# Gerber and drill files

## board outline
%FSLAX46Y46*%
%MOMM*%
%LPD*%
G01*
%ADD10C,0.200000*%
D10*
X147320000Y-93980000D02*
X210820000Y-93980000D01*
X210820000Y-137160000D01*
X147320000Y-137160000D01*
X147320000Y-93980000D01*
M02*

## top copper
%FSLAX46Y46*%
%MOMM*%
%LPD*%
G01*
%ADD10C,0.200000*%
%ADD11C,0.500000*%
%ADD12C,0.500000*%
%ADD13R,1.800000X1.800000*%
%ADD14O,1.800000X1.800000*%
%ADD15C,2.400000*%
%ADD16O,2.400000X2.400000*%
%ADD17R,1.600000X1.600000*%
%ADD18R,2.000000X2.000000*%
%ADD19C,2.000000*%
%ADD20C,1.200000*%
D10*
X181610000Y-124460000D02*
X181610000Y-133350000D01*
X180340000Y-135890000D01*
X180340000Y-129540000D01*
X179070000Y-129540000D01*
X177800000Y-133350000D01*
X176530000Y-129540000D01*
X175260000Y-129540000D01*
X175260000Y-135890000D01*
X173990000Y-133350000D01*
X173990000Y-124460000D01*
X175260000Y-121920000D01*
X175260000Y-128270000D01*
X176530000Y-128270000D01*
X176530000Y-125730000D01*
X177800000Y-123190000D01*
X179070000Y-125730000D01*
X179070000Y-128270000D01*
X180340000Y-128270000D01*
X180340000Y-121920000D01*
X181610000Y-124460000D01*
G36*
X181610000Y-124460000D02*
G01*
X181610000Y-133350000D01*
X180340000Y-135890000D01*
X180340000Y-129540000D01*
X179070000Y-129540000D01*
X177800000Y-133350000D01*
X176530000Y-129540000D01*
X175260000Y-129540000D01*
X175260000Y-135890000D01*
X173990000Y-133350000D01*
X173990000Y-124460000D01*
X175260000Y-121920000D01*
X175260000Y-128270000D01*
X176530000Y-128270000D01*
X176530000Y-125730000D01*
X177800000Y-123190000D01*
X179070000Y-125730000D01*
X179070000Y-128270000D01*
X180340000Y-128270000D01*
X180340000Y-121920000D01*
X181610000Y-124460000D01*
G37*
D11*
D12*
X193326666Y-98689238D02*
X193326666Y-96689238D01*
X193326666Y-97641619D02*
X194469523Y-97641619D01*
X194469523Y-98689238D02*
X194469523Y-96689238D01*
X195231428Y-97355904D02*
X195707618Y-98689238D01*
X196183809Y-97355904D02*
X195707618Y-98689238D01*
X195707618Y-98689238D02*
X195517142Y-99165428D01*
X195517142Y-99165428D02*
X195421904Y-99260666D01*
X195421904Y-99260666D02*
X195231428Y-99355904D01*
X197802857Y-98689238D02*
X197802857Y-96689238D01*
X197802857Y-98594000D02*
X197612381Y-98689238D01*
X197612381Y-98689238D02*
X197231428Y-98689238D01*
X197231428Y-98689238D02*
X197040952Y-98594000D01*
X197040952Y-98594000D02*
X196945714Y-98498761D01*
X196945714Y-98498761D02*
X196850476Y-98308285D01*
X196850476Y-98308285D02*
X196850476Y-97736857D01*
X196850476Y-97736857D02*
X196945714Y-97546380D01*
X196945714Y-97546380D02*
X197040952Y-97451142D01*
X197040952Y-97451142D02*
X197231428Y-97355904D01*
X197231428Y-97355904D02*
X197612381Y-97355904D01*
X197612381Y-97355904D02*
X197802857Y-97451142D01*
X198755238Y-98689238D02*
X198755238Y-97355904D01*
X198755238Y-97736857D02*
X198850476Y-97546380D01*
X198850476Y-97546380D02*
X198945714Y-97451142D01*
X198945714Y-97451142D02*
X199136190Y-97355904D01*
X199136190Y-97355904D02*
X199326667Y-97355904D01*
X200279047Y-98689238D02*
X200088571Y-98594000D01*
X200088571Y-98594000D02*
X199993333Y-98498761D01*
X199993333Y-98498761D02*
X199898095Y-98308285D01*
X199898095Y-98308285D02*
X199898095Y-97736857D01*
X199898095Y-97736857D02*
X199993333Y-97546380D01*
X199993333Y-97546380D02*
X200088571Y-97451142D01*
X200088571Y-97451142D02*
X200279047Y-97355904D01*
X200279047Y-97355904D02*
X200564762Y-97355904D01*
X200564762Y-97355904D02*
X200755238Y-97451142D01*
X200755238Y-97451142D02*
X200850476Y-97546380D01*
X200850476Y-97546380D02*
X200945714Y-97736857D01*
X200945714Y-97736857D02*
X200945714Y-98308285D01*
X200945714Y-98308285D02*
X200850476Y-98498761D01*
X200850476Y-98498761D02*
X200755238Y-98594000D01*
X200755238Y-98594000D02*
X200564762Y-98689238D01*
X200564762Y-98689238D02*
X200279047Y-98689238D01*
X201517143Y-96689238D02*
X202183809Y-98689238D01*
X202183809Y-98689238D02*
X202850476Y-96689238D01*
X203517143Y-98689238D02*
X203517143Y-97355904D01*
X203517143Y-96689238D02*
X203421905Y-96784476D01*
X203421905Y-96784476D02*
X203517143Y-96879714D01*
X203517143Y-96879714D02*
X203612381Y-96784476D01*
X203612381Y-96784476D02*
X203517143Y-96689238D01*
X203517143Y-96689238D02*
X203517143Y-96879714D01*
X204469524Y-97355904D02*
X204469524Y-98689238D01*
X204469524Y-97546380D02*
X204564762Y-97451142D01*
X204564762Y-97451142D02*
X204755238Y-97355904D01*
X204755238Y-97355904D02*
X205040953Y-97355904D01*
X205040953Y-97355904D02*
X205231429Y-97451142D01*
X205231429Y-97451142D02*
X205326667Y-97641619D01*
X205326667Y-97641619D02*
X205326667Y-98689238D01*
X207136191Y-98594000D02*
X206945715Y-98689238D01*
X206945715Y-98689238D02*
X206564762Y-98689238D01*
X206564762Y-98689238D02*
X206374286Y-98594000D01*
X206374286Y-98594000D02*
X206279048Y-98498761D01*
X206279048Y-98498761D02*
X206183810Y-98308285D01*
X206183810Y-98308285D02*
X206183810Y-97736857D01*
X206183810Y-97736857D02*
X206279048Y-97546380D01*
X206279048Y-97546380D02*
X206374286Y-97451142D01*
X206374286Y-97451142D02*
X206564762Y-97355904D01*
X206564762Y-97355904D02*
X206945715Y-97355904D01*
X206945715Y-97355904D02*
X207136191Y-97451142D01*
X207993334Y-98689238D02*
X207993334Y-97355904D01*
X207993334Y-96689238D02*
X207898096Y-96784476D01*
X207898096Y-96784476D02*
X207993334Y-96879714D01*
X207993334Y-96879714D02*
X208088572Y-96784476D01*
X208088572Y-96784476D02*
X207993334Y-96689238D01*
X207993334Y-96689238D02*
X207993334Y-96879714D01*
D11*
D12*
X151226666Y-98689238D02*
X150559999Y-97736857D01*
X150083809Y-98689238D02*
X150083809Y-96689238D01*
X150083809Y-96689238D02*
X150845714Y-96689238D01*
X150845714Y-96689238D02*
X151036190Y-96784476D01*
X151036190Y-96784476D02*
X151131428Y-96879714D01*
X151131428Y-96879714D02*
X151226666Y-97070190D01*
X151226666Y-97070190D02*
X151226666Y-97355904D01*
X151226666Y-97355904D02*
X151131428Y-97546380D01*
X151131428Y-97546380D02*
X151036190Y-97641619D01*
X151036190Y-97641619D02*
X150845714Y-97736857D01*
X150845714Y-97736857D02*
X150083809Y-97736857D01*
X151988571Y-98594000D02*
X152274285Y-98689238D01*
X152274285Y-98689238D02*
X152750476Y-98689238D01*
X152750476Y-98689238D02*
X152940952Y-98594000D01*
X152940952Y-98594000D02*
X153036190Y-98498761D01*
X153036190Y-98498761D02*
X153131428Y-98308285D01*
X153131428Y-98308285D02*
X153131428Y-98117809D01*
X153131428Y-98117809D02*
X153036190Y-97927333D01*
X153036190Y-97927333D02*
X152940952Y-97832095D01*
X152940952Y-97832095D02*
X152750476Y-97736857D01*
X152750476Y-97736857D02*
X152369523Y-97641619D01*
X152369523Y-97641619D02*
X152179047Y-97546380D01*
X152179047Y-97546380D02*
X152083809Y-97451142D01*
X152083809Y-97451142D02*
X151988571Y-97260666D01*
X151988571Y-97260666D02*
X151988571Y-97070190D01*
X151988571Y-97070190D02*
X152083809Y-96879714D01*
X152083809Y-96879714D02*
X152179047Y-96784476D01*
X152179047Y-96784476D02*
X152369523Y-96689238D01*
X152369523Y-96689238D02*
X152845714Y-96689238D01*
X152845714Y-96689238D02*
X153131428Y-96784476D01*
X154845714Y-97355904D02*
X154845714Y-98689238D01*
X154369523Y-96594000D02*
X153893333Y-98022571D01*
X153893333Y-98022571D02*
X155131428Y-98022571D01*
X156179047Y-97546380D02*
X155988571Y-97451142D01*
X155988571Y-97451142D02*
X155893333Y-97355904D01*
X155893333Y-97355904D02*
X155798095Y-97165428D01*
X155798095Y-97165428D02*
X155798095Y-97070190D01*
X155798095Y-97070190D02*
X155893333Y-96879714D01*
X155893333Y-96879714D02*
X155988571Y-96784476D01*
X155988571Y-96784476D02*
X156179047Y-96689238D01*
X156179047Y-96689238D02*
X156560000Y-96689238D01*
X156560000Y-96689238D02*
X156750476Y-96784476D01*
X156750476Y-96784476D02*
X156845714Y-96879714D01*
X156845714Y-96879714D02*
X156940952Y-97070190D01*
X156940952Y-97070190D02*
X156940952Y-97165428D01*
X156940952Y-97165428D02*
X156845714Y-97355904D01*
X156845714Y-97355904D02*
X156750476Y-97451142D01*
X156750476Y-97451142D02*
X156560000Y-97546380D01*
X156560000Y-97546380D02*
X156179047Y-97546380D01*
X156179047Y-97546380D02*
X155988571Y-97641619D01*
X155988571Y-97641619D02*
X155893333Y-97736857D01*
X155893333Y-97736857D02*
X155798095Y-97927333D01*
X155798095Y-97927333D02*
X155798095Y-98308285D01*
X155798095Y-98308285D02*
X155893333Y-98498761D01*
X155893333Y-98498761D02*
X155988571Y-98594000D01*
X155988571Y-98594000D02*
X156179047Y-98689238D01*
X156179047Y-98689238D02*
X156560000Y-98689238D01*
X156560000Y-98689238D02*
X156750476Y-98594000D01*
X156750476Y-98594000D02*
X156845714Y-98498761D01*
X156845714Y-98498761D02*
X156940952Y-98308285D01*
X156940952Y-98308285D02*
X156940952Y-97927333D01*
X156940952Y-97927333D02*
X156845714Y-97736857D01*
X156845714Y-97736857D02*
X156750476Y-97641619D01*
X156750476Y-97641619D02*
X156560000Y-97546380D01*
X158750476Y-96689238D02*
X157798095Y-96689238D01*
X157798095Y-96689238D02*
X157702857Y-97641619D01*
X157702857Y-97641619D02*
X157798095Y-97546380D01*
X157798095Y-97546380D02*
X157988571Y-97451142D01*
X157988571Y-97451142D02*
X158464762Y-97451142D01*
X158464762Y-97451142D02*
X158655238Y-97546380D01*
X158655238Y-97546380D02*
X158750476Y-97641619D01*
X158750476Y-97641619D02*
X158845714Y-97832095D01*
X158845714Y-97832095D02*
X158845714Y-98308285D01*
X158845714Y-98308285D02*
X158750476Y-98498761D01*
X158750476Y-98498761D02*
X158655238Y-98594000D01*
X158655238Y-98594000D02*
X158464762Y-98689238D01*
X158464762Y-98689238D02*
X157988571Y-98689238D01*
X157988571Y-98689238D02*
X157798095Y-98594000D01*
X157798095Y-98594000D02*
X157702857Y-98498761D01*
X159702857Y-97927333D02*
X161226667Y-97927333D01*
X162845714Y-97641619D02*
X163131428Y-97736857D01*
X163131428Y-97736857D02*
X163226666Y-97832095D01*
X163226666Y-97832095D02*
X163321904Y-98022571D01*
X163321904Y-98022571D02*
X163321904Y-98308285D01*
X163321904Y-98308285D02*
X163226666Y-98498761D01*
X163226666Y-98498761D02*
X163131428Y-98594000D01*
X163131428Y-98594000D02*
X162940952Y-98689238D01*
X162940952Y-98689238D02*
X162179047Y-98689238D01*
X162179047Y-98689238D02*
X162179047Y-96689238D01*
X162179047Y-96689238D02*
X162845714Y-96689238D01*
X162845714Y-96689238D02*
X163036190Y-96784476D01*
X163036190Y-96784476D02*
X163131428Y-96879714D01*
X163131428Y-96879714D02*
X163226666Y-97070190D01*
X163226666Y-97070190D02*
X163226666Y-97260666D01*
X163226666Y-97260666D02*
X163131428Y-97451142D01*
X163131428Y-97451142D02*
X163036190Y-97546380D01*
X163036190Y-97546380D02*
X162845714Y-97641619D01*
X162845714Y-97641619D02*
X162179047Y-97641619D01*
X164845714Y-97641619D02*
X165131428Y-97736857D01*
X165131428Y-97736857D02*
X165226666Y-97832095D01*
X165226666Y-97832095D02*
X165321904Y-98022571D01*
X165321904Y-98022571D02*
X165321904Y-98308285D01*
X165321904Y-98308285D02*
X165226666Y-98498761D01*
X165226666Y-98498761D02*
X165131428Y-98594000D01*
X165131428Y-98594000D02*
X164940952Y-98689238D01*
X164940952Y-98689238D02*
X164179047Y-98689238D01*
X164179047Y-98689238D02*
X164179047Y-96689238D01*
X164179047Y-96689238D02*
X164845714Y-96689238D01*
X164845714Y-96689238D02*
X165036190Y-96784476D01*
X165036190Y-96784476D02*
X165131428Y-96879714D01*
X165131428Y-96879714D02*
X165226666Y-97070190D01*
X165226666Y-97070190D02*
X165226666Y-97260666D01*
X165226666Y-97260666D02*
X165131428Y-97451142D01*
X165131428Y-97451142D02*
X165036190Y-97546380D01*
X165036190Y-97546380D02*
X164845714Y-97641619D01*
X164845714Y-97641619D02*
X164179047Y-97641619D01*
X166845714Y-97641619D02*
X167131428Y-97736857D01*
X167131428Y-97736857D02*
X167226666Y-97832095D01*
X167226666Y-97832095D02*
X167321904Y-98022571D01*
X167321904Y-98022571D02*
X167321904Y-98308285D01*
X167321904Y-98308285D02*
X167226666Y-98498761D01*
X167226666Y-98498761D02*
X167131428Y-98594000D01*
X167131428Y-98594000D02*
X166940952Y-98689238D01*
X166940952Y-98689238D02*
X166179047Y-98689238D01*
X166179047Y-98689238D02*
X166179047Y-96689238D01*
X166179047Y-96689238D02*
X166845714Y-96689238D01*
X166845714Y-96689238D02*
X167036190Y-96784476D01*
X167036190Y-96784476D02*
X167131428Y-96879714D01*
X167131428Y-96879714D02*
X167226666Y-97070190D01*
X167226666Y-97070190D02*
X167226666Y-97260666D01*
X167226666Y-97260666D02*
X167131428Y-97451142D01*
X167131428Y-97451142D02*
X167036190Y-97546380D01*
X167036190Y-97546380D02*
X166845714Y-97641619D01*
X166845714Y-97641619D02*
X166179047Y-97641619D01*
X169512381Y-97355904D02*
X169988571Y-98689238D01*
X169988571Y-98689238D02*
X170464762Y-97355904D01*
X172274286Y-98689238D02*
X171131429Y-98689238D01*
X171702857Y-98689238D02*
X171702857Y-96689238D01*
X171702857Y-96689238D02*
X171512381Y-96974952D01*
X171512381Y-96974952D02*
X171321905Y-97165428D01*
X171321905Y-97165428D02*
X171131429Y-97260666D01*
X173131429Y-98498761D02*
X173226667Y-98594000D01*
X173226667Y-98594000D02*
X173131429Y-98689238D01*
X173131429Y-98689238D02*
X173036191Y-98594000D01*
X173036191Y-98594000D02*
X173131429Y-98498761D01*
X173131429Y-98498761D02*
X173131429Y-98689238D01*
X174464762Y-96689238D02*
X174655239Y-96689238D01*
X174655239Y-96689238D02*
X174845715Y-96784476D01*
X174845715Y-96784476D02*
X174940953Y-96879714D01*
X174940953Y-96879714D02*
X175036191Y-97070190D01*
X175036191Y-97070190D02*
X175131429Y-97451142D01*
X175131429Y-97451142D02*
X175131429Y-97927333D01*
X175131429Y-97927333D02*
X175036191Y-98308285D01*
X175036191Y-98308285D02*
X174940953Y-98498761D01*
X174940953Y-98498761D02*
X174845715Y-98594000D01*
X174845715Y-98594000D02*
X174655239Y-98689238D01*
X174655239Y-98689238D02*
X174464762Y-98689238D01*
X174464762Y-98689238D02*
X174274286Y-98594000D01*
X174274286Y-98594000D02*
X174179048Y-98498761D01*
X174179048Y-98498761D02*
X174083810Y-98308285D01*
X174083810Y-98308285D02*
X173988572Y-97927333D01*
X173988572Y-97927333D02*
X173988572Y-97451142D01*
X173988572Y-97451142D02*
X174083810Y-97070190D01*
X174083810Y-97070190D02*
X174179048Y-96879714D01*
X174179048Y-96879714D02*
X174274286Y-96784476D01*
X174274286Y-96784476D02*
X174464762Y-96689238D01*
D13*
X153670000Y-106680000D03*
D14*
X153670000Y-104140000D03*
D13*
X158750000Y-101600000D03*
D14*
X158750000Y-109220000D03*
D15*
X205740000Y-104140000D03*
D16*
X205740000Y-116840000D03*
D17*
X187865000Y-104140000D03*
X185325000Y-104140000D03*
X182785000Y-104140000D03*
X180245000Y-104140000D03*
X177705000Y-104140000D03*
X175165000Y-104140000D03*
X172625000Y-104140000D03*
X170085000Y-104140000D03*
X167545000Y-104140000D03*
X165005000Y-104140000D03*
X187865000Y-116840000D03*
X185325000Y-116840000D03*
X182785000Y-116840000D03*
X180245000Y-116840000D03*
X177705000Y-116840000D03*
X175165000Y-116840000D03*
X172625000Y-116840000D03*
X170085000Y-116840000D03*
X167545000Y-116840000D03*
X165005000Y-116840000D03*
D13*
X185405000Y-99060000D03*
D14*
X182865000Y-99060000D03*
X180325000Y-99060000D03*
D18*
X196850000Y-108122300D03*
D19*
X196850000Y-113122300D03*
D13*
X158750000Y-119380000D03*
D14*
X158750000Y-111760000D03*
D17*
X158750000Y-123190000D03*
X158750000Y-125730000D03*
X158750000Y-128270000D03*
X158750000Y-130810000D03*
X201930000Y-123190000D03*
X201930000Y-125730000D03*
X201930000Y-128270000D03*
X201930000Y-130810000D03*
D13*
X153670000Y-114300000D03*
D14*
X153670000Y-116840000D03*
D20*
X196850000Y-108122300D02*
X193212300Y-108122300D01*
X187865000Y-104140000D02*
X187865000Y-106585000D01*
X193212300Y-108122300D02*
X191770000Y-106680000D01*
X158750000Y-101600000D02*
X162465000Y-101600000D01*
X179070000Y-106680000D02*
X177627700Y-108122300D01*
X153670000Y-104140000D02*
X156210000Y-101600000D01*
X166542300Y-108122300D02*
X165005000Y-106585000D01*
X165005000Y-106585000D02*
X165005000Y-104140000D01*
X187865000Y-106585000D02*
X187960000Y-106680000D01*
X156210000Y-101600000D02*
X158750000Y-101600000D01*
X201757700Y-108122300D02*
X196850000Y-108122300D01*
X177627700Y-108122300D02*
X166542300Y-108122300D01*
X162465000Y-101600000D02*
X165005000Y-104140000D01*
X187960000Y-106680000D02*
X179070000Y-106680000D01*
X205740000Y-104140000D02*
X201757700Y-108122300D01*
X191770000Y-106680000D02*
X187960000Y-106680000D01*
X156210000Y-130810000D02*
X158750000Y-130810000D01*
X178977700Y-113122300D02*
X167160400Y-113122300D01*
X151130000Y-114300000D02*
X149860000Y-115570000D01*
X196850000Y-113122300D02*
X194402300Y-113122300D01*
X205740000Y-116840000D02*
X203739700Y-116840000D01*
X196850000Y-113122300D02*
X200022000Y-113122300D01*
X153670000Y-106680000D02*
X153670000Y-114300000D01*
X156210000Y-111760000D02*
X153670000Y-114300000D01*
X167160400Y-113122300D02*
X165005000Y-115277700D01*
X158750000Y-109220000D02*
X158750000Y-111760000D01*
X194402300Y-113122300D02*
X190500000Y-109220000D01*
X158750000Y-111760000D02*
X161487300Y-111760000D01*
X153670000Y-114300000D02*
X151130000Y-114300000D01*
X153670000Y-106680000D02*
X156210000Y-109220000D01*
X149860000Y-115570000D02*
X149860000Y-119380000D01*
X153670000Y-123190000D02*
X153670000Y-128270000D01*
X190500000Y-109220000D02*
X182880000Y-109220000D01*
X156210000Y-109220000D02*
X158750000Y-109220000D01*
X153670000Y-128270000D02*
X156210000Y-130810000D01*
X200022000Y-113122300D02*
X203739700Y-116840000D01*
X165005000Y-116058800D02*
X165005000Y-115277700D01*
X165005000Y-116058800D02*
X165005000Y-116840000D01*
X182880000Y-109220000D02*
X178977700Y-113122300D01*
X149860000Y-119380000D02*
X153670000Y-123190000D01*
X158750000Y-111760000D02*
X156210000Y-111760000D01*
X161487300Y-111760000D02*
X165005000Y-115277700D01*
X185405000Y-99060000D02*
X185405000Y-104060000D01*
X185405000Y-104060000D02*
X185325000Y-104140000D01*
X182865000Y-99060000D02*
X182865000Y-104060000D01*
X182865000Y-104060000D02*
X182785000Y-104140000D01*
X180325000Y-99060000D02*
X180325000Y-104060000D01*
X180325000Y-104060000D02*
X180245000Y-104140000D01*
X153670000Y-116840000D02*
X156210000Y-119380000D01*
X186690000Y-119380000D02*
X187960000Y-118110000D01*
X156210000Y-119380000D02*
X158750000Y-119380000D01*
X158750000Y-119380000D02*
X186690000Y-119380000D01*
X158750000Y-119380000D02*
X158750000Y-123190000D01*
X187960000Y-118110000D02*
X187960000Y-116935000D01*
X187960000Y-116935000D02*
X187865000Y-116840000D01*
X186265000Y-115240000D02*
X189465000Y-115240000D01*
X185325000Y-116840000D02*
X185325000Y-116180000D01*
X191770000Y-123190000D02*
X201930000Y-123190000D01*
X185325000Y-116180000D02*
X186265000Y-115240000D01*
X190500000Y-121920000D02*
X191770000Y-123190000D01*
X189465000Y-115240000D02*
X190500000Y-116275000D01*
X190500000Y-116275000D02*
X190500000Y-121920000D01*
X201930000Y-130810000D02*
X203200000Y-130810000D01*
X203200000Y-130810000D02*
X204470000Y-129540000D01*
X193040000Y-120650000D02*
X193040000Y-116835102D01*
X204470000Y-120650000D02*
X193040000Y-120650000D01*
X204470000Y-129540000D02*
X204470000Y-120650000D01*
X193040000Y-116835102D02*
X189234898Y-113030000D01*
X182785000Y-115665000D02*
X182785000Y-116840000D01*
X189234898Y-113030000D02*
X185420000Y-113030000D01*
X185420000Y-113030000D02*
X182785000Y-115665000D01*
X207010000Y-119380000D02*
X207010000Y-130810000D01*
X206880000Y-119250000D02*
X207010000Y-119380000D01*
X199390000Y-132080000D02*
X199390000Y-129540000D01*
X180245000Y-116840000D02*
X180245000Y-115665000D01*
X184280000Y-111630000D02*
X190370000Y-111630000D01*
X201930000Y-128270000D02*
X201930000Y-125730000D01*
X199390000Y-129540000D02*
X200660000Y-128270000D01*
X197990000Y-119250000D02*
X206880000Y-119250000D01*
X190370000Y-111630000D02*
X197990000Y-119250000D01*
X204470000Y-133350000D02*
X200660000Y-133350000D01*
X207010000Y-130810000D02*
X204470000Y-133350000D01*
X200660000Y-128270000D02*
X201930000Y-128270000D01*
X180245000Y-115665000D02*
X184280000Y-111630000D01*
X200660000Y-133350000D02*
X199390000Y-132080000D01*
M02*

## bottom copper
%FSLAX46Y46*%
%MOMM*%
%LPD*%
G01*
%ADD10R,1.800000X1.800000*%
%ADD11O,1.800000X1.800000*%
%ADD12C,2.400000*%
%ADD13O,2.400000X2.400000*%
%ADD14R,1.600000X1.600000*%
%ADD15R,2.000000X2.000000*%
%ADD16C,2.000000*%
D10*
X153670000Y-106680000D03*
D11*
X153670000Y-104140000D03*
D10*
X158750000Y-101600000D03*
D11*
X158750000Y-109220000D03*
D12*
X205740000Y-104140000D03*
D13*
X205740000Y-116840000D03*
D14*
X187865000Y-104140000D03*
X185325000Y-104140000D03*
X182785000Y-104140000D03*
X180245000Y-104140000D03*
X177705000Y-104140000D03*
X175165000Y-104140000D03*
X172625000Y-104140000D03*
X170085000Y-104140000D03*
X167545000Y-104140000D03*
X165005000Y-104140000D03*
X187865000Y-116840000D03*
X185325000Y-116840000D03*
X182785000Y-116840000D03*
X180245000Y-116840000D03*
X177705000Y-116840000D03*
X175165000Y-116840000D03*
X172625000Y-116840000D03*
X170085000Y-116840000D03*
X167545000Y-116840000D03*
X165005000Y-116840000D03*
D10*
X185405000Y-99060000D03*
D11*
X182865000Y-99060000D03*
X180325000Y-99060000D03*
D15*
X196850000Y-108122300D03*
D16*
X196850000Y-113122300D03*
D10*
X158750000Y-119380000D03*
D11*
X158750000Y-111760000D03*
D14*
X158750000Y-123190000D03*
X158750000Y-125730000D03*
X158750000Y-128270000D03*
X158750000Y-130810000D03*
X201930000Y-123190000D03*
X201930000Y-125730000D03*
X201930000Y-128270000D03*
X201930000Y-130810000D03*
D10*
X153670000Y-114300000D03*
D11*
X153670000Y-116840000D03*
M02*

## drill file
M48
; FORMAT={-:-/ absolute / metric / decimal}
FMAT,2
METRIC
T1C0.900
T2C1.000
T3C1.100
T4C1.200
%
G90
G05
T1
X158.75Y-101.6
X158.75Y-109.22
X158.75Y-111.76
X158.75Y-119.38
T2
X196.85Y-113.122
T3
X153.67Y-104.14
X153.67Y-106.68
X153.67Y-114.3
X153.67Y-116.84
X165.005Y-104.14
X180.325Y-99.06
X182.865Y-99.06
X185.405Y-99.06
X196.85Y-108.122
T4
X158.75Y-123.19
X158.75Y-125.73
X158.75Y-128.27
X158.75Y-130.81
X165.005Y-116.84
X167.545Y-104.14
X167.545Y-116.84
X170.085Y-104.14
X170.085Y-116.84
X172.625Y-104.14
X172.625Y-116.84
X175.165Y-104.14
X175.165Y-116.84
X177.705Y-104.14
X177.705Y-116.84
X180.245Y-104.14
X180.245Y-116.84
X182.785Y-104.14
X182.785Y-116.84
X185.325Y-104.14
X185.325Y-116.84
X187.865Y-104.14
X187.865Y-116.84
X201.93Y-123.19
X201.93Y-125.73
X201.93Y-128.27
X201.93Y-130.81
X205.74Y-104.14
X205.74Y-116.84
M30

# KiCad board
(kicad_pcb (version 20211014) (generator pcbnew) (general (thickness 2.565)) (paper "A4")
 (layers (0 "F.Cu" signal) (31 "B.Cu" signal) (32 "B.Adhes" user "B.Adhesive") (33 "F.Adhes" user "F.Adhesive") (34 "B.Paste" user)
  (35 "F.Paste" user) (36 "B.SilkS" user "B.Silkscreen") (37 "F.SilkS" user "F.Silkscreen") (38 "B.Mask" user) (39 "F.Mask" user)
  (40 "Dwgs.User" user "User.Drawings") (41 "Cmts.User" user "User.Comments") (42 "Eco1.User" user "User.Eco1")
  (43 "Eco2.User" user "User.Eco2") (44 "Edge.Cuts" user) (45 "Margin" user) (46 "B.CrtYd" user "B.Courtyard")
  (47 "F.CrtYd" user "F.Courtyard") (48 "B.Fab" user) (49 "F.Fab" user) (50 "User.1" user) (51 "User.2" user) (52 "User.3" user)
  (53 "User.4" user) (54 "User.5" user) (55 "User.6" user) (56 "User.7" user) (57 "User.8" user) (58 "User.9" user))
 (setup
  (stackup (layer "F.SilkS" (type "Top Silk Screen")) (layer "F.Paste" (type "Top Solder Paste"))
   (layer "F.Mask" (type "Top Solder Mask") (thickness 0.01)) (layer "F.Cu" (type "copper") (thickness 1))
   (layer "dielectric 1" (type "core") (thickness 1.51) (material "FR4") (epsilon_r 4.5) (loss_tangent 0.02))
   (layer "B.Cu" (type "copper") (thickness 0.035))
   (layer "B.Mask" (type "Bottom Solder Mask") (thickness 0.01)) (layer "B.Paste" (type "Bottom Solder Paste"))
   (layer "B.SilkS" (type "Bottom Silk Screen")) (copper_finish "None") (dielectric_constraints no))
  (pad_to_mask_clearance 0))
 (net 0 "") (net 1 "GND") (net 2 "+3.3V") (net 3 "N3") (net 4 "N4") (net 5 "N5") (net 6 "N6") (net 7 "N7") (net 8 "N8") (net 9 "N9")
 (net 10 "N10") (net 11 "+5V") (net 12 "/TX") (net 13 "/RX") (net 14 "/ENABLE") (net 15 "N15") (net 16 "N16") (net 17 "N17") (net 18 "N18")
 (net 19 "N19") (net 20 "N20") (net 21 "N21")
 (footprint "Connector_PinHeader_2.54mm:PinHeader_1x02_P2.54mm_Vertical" (layer "F.Cu") (at 153.67 106.68 180)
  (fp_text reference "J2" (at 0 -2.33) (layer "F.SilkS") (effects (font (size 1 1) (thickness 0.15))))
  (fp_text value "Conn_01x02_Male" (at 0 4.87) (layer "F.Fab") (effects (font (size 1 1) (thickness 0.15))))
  (pad "1" thru_hole rect (at 0 0 180) (size 1.8 1.8) (drill 1.1) (layers *.Cu *.Mask) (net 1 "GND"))
  (pad "2" thru_hole oval (at 0 2.54 180) (size 1.8 1.8) (drill 1.1) (layers *.Cu *.Mask) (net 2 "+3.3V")))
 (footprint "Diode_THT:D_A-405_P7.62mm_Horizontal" (layer "F.Cu") (at 158.75 101.6 -90)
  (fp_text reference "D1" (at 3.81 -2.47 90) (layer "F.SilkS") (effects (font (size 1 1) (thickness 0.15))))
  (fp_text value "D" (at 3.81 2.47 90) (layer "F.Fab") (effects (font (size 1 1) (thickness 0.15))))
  (pad "1" thru_hole rect (at 0 0 270) (size 1.8 1.8) (drill 0.9) (layers *.Cu *.Mask) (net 2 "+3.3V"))
  (pad "2" thru_hole oval (at 7.62 0 270) (size 1.8 1.8) (drill 0.9) (layers *.Cu *.Mask) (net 1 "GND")))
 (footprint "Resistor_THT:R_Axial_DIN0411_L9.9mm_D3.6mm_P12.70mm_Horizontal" (layer "F.Cu") (at 205.74 104.14 -90)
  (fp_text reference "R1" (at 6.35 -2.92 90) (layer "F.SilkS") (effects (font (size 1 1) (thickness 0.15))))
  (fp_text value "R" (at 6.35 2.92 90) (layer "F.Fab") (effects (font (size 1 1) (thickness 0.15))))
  (pad "1" thru_hole circle (at 0 0 270) (size 2.4 2.4) (drill 1.2) (layers *.Cu *.Mask) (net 2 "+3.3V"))
  (pad "2" thru_hole oval (at 12.7 0 270) (size 2.4 2.4) (drill 1.2) (layers *.Cu *.Mask) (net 1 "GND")))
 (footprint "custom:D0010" (layer "F.Cu") (at 190.405 109.22 -90)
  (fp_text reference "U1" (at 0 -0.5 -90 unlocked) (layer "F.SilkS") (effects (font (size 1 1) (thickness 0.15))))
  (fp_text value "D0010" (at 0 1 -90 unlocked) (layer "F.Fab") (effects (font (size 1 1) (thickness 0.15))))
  (pad "1" thru_hole rect (at -5.08 2.54 270) (size 1.6 1.6) (drill 1.2) (layers *.Cu *.Mask) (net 2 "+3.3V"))
  (pad "2" thru_hole rect (at -5.08 5.08 270) (size 1.6 1.6) (drill 1.2) (layers *.Cu *.Mask) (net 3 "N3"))
  (pad "3" thru_hole rect (at -5.08 7.62 270) (size 1.6 1.6) (drill 1.2) (layers *.Cu *.Mask) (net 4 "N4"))
  (pad "4" thru_hole rect (at -5.08 10.16 270) (size 1.6 1.6) (drill 1.2) (layers *.Cu *.Mask) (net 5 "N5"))
  (pad "5" thru_hole rect (at -5.08 12.7 270) (size 1.6 1.6) (drill 1.2) (layers *.Cu *.Mask) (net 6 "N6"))
  (pad "6" thru_hole rect (at -5.08 15.24 270) (size 1.6 1.6) (drill 1.2) (layers *.Cu *.Mask) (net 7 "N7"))
  (pad "7" thru_hole rect (at -5.08 17.78 270) (size 1.6 1.6) (drill 1.2) (layers *.Cu *.Mask) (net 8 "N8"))
  (pad "8" thru_hole rect (at -5.08 20.32 270) (size 1.6 1.6) (drill 1.2) (layers *.Cu *.Mask) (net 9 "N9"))
  (pad "9" thru_hole rect (at -5.08 22.86 270) (size 1.6 1.6) (drill 1.2) (layers *.Cu *.Mask) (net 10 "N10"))
  (pad "10" thru_hole rect (at -5.08 25.4 270) (size 1.6 1.6) (drill 1.1) (layers *.Cu *.Mask) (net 2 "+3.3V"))
  (pad "11" thru_hole rect (at 7.62 2.54 270) (size 1.6 1.6) (drill 1.2) (layers *.Cu *.Mask) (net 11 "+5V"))
  (pad "12" thru_hole rect (at 7.62 5.08 270) (size 1.6 1.6) (drill 1.2) (layers *.Cu *.Mask) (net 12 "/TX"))
  (pad "13" thru_hole rect (at 7.62 7.62 270) (size 1.6 1.6) (drill 1.2) (layers *.Cu *.Mask) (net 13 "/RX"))
  (pad "14" thru_hole rect (at 7.62 10.16 270) (size 1.6 1.6) (drill 1.2) (layers *.Cu *.Mask) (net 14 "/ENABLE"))
  (pad "15" thru_hole rect (at 7.62 12.7 270) (size 1.6 1.6) (drill 1.2) (layers *.Cu *.Mask) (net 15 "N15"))
  (pad "16" thru_hole rect (at 7.62 15.24 270) (size 1.6 1.6) (drill 1.2) (layers *.Cu *.Mask) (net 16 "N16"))
  (pad "17" thru_hole rect (at 7.62 17.78 270) (size 1.6 1.6) (drill 1.2) (layers *.Cu *.Mask) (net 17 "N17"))
  (pad "18" thru_hole rect (at 7.62 20.32 270) (size 1.6 1.6) (drill 1.2) (layers *.Cu *.Mask) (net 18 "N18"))
  (pad "19" thru_hole rect (at 7.62 22.86 270) (size 1.6 1.6) (drill 1.2) (layers *.Cu *.Mask) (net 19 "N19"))
  (pad "20" thru_hole rect (at 7.62 25.4 270) (size 1.6 1.6) (drill 1.2) (layers *.Cu *.Mask) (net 1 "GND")))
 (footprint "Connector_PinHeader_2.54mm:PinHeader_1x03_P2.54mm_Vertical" (layer "F.Cu") (at 185.405 99.06 -90)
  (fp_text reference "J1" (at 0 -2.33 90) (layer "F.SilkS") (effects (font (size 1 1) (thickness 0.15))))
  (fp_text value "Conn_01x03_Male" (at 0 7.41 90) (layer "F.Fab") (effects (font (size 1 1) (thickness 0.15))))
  (pad "1" thru_hole rect (at 0 0 270) (size 1.8 1.8) (drill 1.1) (layers *.Cu *.Mask) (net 3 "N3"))
  (pad "2" thru_hole oval (at 0 2.54 270) (size 1.8 1.8) (drill 1.1) (layers *.Cu *.Mask) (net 4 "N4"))
  (pad "3" thru_hole oval (at 0 5.08 270) (size 1.8 1.8) (drill 1.1) (layers *.Cu *.Mask) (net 5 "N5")))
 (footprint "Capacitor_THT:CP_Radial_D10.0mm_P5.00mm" (layer "F.Cu") (at 196.85 108.1223 -90)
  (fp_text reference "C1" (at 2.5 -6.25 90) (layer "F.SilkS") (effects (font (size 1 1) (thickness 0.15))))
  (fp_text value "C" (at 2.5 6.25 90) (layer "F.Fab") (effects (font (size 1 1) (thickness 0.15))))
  (pad "1" thru_hole rect (at 0 0 270) (size 2 2) (drill 1.1) (layers *.Cu *.Mask) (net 2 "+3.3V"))
  (pad "2" thru_hole circle (at 5 0 270) (size 2 2) (drill 1) (layers *.Cu *.Mask) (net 1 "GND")))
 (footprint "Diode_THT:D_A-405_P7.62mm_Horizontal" (layer "F.Cu") (at 158.75 119.38 90)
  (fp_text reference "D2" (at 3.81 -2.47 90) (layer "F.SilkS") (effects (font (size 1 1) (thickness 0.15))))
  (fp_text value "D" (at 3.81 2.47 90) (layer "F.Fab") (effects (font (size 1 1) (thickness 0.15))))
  (pad "1" thru_hole rect (at 0 0 90) (size 1.8 1.8) (drill 0.9) (layers *.Cu *.Mask) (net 11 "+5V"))
  (pad "2" thru_hole oval (at 7.62 0 90) (size 1.8 1.8) (drill 0.9) (layers *.Cu *.Mask) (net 1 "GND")))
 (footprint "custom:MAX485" (layer "F.Cu") (at 163.83 118.11)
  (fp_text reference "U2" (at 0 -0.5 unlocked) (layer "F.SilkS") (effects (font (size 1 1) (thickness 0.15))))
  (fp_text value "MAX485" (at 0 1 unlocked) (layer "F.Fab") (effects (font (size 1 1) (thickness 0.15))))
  (pad "1" thru_hole rect (at -5.08 5.08) (size 1.6 1.6) (drill 1.2) (layers *.Cu *.Mask) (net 11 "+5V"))
  (pad "2" thru_hole rect (at -5.08 7.62) (size 1.6 1.6) (drill 1.2) (layers *.Cu *.Mask) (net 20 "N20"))
  (pad "3" thru_hole rect (at -5.08 10.16) (size 1.6 1.6) (drill 1.2) (layers *.Cu *.Mask) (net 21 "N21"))
  (pad "4" thru_hole rect (at -5.08 12.7) (size 1.6 1.6) (drill 1.2) (layers *.Cu *.Mask) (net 1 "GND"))
  (pad "5" thru_hole rect (at 38.1 5.08) (size 1.6 1.6) (drill 1.2) (layers *.Cu *.Mask) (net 12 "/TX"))
  (pad "6" thru_hole rect (at 38.1 7.62) (size 1.6 1.6) (drill 1.2) (layers *.Cu *.Mask) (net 14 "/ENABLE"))
  (pad "7" thru_hole rect (at 38.1 10.16) (size 1.6 1.6) (drill 1.2) (layers *.Cu *.Mask) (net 14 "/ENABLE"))
  (pad "8" thru_hole rect (at 38.1 12.7) (size 1.6 1.6) (drill 1.2) (layers *.Cu *.Mask) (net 13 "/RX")))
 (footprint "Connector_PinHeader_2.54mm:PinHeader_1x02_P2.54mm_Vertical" (layer "F.Cu") (at 153.67 114.3)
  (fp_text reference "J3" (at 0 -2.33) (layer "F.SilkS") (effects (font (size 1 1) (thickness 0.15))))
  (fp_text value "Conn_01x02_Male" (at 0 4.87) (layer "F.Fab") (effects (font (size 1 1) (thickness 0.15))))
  (pad "1" thru_hole rect (at 0 0) (size 1.8 1.8) (drill 1.1) (layers *.Cu *.Mask) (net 1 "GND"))
  (pad "2" thru_hole oval (at 0 2.54) (size 1.8 1.8) (drill 1.1) (layers *.Cu *.Mask) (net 11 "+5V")))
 (gr_poly
  (pts (xy 181.61 124.46) (xy 181.61 133.35) (xy 180.34 135.89) (xy 180.34 129.54) (xy 179.07 129.54) (xy 177.8 133.35) (xy 176.53 129.54)
   (xy 175.26 129.54) (xy 175.26 135.89) (xy 173.99 133.35) (xy 173.99 124.46) (xy 175.26 121.92) (xy 175.26 128.27) (xy 176.53 128.27)
   (xy 176.53 125.73) (xy 177.8 123.19) (xy 179.07 125.73) (xy 179.07 128.27) (xy 180.34 128.27) (xy 180.34 121.92))
  (layer "F.Cu") (width 0.2) (fill solid))
 (gr_rect (start 147.32 93.98) (end 210.82 137.16) (layer "Edge.Cuts") (width 0.2) (fill none))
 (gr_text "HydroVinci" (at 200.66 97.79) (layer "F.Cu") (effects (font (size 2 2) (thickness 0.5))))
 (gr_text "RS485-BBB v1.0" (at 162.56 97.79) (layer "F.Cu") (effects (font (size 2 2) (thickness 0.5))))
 (segment (start 196.85 108.1223) (end 193.2123 108.1223) (width 1.2) (layer "F.Cu") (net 2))
 (segment (start 187.865 104.14) (end 187.865 106.585) (width 1.2) (layer "F.Cu") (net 2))
 (segment (start 193.2123 108.1223) (end 191.77 106.68) (width 1.2) (layer "F.Cu") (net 2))
 (segment (start 158.75 101.6) (end 162.465 101.6) (width 1.2) (layer "F.Cu") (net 2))
 (segment (start 179.07 106.68) (end 177.6277 108.1223) (width 1.2) (layer "F.Cu") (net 2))
 (segment (start 153.67 104.14) (end 156.21 101.6) (width 1.2) (layer "F.Cu") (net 2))
 (segment (start 166.5423 108.1223) (end 165.005 106.585) (width 1.2) (layer "F.Cu") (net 2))
 (segment (start 165.005 106.585) (end 165.005 104.14) (width 1.2) (layer "F.Cu") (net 2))
 (segment (start 187.865 106.585) (end 187.96 106.68) (width 1.2) (layer "F.Cu") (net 2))
 (segment (start 156.21 101.6) (end 158.75 101.6) (width 1.2) (layer "F.Cu") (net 2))
 (segment (start 201.7577 108.1223) (end 196.85 108.1223) (width 1.2) (layer "F.Cu") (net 2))
 (segment (start 177.6277 108.1223) (end 166.5423 108.1223) (width 1.2) (layer "F.Cu") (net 2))
 (segment (start 162.465 101.6) (end 165.005 104.14) (width 1.2) (layer "F.Cu") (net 2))
 (segment (start 187.96 106.68) (end 179.07 106.68) (width 1.2) (layer "F.Cu") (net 2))
 (segment (start 205.74 104.14) (end 201.7577 108.1223) (width 1.2) (layer "F.Cu") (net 2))
 (segment (start 191.77 106.68) (end 187.96 106.68) (width 1.2) (layer "F.Cu") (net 2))
 (segment (start 156.21 130.81) (end 158.75 130.81) (width 1.2) (layer "F.Cu") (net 1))
 (segment (start 178.9777 113.1223) (end 167.1604 113.1223) (width 1.2) (layer "F.Cu") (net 1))
 (segment (start 151.13 114.3) (end 149.86 115.57) (width 1.2) (layer "F.Cu") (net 1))
 (segment (start 196.85 113.1223) (end 194.4023 113.1223) (width 1.2) (layer "F.Cu") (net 1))
 (segment (start 205.74 116.84) (end 203.7397 116.84) (width 1.2) (layer "F.Cu") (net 1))
 (segment (start 196.85 113.1223) (end 200.022 113.1223) (width 1.2) (layer "F.Cu") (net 1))
 (segment (start 153.67 106.68) (end 153.67 114.3) (width 1.2) (layer "F.Cu") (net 1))
 (segment (start 156.21 111.76) (end 153.67 114.3) (width 1.2) (layer "F.Cu") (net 1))
 (segment (start 167.1604 113.1223) (end 165.005 115.2777) (width 1.2) (layer "F.Cu") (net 1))
 (segment (start 158.75 109.22) (end 158.75 111.76) (width 1.2) (layer "F.Cu") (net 1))
 (segment (start 194.4023 113.1223) (end 190.5 109.22) (width 1.2) (layer "F.Cu") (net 1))
 (segment (start 158.75 111.76) (end 161.4873 111.76) (width 1.2) (layer "F.Cu") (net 1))
 (segment (start 153.67 114.3) (end 151.13 114.3) (width 1.2) (layer "F.Cu") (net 1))
 (segment (start 153.67 106.68) (end 156.21 109.22) (width 1.2) (layer "F.Cu") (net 1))
 (segment (start 149.86 115.57) (end 149.86 119.38) (width 1.2) (layer "F.Cu") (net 1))
 (segment (start 153.67 123.19) (end 153.67 128.27) (width 1.2) (layer "F.Cu") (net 1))
 (segment (start 190.5 109.22) (end 182.88 109.22) (width 1.2) (layer "F.Cu") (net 1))
 (segment (start 156.21 109.22) (end 158.75 109.22) (width 1.2) (layer "F.Cu") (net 1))
 (segment (start 153.67 128.27) (end 156.21 130.81) (width 1.2) (layer "F.Cu") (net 1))
 (segment (start 200.022 113.1223) (end 203.7397 116.84) (width 1.2) (layer "F.Cu") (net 1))
 (segment (start 165.005 116.0588) (end 165.005 115.2777) (width 1.2) (layer "F.Cu") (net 1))
 (segment (start 165.005 116.0588) (end 165.005 116.84) (width 1.2) (layer "F.Cu") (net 1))
 (segment (start 182.88 109.22) (end 178.9777 113.1223) (width 1.2) (layer "F.Cu") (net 1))
 (segment (start 149.86 119.38) (end 153.67 123.19) (width 1.2) (layer "F.Cu") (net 1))
 (segment (start 158.75 111.76) (end 156.21 111.76) (width 1.2) (layer "F.Cu") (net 1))
 (segment (start 161.4873 111.76) (end 165.005 115.2777) (width 1.2) (layer "F.Cu") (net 1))
 (segment (start 185.405 99.06) (end 185.405 104.06) (width 1.2) (layer "F.Cu") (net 3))
 (segment (start 185.405 104.06) (end 185.325 104.14) (width 1.2) (layer "F.Cu") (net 3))
 (segment (start 182.865 99.06) (end 182.865 104.06) (width 1.2) (layer "F.Cu") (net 4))
 (segment (start 182.865 104.06) (end 182.785 104.14) (width 1.2) (layer "F.Cu") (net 4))
 (segment (start 180.325 99.06) (end 180.325 104.06) (width 1.2) (layer "F.Cu") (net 5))
 (segment (start 180.325 104.06) (end 180.245 104.14) (width 1.2) (layer "F.Cu") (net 5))
 (segment (start 153.67 116.84) (end 156.21 119.38) (width 1.2) (layer "F.Cu") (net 11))
 (segment (start 186.69 119.38) (end 187.96 118.11) (width 1.2) (layer "F.Cu") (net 11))
 (segment (start 156.21 119.38) (end 158.75 119.38) (width 1.2) (layer "F.Cu") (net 11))
 (segment (start 158.75 119.38) (end 186.69 119.38) (width 1.2) (layer "F.Cu") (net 11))
 (segment (start 158.75 119.38) (end 158.75 123.19) (width 1.2) (layer "F.Cu") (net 11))
 (segment (start 187.96 118.11) (end 187.96 116.935) (width 1.2) (layer "F.Cu") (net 11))
 (segment (start 187.96 116.935) (end 187.865 116.84) (width 1.2) (layer "F.Cu") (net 11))
 (segment (start 186.265 115.24) (end 189.465 115.24) (width 1.2) (layer "F.Cu") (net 12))
 (segment (start 185.325 116.84) (end 185.325 116.18) (width 1.2) (layer "F.Cu") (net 12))
 (segment (start 191.77 123.19) (end 201.93 123.19) (width 1.2) (layer "F.Cu") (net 12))
 (segment (start 185.325 116.18) (end 186.265 115.24) (width 1.2) (layer "F.Cu") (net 12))
 (segment (start 190.5 121.92) (end 191.77 123.19) (width 1.2) (layer "F.Cu") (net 12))
 (segment (start 189.465 115.24) (end 190.5 116.275) (width 1.2) (layer "F.Cu") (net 12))
 (segment (start 190.5 116.275) (end 190.5 121.92) (width 1.2) (layer "F.Cu") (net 12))
 (segment (start 201.93 130.81) (end 203.2 130.81) (width 1.2) (layer "F.Cu") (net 13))
 (segment (start 203.2 130.81) (end 204.47 129.54) (width 1.2) (layer "F.Cu") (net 13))
 (segment (start 193.04 120.65) (end 193.04 116.835102) (width 1.2) (layer "F.Cu") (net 13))
 (segment (start 204.47 120.65) (end 193.04 120.65) (width 1.2) (layer "F.Cu") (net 13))
 (segment (start 204.47 129.54) (end 204.47 120.65) (width 1.2) (layer "F.Cu") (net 13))
 (segment (start 193.04 116.835102) (end 189.234898 113.03) (width 1.2) (layer "F.Cu") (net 13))
 (segment (start 182.785 115.665) (end 182.785 116.84) (width 1.2) (layer "F.Cu") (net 13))
 (segment (start 189.234898 113.03) (end 185.42 113.03) (width 1.2) (layer "F.Cu") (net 13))
 (segment (start 185.42 113.03) (end 182.785 115.665) (width 1.2) (layer "F.Cu") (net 13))
 (segment (start 207.01 119.38) (end 207.01 130.81) (width 1.2) (layer "F.Cu") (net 14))
 (segment (start 206.88 119.25) (end 207.01 119.38) (width 1.2) (layer "F.Cu") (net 14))
 (segment (start 199.39 132.08) (end 199.39 129.54) (width 1.2) (layer "F.Cu") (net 14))
 (segment (start 180.245 116.84) (end 180.245 115.665) (width 1.2) (layer "F.Cu") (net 14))
 (segment (start 184.28 111.63) (end 190.37 111.63) (width 1.2) (layer "F.Cu") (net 14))
 (segment (start 201.93 128.27) (end 201.93 125.73) (width 1.2) (layer "F.Cu") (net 14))
 (segment (start 199.39 129.54) (end 200.66 128.27) (width 1.2) (layer "F.Cu") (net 14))
 (segment (start 197.99 119.25) (end 206.88 119.25) (width 1.2) (layer "F.Cu") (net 14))
 (segment (start 190.37 111.63) (end 197.99 119.25) (width 1.2) (layer "F.Cu") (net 14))
 (segment (start 204.47 133.35) (end 200.66 133.35) (width 1.2) (layer "F.Cu") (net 14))
 (segment (start 207.01 130.81) (end 204.47 133.35) (width 1.2) (layer "F.Cu") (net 14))
 (segment (start 200.66 128.27) (end 201.93 128.27) (width 1.2) (layer "F.Cu") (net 14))
 (segment (start 180.245 115.665) (end 184.28 111.63) (width 1.2) (layer "F.Cu") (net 14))
 (segment (start 200.66 133.35) (end 199.39 132.08) (width 1.2) (layer "F.Cu") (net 14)))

